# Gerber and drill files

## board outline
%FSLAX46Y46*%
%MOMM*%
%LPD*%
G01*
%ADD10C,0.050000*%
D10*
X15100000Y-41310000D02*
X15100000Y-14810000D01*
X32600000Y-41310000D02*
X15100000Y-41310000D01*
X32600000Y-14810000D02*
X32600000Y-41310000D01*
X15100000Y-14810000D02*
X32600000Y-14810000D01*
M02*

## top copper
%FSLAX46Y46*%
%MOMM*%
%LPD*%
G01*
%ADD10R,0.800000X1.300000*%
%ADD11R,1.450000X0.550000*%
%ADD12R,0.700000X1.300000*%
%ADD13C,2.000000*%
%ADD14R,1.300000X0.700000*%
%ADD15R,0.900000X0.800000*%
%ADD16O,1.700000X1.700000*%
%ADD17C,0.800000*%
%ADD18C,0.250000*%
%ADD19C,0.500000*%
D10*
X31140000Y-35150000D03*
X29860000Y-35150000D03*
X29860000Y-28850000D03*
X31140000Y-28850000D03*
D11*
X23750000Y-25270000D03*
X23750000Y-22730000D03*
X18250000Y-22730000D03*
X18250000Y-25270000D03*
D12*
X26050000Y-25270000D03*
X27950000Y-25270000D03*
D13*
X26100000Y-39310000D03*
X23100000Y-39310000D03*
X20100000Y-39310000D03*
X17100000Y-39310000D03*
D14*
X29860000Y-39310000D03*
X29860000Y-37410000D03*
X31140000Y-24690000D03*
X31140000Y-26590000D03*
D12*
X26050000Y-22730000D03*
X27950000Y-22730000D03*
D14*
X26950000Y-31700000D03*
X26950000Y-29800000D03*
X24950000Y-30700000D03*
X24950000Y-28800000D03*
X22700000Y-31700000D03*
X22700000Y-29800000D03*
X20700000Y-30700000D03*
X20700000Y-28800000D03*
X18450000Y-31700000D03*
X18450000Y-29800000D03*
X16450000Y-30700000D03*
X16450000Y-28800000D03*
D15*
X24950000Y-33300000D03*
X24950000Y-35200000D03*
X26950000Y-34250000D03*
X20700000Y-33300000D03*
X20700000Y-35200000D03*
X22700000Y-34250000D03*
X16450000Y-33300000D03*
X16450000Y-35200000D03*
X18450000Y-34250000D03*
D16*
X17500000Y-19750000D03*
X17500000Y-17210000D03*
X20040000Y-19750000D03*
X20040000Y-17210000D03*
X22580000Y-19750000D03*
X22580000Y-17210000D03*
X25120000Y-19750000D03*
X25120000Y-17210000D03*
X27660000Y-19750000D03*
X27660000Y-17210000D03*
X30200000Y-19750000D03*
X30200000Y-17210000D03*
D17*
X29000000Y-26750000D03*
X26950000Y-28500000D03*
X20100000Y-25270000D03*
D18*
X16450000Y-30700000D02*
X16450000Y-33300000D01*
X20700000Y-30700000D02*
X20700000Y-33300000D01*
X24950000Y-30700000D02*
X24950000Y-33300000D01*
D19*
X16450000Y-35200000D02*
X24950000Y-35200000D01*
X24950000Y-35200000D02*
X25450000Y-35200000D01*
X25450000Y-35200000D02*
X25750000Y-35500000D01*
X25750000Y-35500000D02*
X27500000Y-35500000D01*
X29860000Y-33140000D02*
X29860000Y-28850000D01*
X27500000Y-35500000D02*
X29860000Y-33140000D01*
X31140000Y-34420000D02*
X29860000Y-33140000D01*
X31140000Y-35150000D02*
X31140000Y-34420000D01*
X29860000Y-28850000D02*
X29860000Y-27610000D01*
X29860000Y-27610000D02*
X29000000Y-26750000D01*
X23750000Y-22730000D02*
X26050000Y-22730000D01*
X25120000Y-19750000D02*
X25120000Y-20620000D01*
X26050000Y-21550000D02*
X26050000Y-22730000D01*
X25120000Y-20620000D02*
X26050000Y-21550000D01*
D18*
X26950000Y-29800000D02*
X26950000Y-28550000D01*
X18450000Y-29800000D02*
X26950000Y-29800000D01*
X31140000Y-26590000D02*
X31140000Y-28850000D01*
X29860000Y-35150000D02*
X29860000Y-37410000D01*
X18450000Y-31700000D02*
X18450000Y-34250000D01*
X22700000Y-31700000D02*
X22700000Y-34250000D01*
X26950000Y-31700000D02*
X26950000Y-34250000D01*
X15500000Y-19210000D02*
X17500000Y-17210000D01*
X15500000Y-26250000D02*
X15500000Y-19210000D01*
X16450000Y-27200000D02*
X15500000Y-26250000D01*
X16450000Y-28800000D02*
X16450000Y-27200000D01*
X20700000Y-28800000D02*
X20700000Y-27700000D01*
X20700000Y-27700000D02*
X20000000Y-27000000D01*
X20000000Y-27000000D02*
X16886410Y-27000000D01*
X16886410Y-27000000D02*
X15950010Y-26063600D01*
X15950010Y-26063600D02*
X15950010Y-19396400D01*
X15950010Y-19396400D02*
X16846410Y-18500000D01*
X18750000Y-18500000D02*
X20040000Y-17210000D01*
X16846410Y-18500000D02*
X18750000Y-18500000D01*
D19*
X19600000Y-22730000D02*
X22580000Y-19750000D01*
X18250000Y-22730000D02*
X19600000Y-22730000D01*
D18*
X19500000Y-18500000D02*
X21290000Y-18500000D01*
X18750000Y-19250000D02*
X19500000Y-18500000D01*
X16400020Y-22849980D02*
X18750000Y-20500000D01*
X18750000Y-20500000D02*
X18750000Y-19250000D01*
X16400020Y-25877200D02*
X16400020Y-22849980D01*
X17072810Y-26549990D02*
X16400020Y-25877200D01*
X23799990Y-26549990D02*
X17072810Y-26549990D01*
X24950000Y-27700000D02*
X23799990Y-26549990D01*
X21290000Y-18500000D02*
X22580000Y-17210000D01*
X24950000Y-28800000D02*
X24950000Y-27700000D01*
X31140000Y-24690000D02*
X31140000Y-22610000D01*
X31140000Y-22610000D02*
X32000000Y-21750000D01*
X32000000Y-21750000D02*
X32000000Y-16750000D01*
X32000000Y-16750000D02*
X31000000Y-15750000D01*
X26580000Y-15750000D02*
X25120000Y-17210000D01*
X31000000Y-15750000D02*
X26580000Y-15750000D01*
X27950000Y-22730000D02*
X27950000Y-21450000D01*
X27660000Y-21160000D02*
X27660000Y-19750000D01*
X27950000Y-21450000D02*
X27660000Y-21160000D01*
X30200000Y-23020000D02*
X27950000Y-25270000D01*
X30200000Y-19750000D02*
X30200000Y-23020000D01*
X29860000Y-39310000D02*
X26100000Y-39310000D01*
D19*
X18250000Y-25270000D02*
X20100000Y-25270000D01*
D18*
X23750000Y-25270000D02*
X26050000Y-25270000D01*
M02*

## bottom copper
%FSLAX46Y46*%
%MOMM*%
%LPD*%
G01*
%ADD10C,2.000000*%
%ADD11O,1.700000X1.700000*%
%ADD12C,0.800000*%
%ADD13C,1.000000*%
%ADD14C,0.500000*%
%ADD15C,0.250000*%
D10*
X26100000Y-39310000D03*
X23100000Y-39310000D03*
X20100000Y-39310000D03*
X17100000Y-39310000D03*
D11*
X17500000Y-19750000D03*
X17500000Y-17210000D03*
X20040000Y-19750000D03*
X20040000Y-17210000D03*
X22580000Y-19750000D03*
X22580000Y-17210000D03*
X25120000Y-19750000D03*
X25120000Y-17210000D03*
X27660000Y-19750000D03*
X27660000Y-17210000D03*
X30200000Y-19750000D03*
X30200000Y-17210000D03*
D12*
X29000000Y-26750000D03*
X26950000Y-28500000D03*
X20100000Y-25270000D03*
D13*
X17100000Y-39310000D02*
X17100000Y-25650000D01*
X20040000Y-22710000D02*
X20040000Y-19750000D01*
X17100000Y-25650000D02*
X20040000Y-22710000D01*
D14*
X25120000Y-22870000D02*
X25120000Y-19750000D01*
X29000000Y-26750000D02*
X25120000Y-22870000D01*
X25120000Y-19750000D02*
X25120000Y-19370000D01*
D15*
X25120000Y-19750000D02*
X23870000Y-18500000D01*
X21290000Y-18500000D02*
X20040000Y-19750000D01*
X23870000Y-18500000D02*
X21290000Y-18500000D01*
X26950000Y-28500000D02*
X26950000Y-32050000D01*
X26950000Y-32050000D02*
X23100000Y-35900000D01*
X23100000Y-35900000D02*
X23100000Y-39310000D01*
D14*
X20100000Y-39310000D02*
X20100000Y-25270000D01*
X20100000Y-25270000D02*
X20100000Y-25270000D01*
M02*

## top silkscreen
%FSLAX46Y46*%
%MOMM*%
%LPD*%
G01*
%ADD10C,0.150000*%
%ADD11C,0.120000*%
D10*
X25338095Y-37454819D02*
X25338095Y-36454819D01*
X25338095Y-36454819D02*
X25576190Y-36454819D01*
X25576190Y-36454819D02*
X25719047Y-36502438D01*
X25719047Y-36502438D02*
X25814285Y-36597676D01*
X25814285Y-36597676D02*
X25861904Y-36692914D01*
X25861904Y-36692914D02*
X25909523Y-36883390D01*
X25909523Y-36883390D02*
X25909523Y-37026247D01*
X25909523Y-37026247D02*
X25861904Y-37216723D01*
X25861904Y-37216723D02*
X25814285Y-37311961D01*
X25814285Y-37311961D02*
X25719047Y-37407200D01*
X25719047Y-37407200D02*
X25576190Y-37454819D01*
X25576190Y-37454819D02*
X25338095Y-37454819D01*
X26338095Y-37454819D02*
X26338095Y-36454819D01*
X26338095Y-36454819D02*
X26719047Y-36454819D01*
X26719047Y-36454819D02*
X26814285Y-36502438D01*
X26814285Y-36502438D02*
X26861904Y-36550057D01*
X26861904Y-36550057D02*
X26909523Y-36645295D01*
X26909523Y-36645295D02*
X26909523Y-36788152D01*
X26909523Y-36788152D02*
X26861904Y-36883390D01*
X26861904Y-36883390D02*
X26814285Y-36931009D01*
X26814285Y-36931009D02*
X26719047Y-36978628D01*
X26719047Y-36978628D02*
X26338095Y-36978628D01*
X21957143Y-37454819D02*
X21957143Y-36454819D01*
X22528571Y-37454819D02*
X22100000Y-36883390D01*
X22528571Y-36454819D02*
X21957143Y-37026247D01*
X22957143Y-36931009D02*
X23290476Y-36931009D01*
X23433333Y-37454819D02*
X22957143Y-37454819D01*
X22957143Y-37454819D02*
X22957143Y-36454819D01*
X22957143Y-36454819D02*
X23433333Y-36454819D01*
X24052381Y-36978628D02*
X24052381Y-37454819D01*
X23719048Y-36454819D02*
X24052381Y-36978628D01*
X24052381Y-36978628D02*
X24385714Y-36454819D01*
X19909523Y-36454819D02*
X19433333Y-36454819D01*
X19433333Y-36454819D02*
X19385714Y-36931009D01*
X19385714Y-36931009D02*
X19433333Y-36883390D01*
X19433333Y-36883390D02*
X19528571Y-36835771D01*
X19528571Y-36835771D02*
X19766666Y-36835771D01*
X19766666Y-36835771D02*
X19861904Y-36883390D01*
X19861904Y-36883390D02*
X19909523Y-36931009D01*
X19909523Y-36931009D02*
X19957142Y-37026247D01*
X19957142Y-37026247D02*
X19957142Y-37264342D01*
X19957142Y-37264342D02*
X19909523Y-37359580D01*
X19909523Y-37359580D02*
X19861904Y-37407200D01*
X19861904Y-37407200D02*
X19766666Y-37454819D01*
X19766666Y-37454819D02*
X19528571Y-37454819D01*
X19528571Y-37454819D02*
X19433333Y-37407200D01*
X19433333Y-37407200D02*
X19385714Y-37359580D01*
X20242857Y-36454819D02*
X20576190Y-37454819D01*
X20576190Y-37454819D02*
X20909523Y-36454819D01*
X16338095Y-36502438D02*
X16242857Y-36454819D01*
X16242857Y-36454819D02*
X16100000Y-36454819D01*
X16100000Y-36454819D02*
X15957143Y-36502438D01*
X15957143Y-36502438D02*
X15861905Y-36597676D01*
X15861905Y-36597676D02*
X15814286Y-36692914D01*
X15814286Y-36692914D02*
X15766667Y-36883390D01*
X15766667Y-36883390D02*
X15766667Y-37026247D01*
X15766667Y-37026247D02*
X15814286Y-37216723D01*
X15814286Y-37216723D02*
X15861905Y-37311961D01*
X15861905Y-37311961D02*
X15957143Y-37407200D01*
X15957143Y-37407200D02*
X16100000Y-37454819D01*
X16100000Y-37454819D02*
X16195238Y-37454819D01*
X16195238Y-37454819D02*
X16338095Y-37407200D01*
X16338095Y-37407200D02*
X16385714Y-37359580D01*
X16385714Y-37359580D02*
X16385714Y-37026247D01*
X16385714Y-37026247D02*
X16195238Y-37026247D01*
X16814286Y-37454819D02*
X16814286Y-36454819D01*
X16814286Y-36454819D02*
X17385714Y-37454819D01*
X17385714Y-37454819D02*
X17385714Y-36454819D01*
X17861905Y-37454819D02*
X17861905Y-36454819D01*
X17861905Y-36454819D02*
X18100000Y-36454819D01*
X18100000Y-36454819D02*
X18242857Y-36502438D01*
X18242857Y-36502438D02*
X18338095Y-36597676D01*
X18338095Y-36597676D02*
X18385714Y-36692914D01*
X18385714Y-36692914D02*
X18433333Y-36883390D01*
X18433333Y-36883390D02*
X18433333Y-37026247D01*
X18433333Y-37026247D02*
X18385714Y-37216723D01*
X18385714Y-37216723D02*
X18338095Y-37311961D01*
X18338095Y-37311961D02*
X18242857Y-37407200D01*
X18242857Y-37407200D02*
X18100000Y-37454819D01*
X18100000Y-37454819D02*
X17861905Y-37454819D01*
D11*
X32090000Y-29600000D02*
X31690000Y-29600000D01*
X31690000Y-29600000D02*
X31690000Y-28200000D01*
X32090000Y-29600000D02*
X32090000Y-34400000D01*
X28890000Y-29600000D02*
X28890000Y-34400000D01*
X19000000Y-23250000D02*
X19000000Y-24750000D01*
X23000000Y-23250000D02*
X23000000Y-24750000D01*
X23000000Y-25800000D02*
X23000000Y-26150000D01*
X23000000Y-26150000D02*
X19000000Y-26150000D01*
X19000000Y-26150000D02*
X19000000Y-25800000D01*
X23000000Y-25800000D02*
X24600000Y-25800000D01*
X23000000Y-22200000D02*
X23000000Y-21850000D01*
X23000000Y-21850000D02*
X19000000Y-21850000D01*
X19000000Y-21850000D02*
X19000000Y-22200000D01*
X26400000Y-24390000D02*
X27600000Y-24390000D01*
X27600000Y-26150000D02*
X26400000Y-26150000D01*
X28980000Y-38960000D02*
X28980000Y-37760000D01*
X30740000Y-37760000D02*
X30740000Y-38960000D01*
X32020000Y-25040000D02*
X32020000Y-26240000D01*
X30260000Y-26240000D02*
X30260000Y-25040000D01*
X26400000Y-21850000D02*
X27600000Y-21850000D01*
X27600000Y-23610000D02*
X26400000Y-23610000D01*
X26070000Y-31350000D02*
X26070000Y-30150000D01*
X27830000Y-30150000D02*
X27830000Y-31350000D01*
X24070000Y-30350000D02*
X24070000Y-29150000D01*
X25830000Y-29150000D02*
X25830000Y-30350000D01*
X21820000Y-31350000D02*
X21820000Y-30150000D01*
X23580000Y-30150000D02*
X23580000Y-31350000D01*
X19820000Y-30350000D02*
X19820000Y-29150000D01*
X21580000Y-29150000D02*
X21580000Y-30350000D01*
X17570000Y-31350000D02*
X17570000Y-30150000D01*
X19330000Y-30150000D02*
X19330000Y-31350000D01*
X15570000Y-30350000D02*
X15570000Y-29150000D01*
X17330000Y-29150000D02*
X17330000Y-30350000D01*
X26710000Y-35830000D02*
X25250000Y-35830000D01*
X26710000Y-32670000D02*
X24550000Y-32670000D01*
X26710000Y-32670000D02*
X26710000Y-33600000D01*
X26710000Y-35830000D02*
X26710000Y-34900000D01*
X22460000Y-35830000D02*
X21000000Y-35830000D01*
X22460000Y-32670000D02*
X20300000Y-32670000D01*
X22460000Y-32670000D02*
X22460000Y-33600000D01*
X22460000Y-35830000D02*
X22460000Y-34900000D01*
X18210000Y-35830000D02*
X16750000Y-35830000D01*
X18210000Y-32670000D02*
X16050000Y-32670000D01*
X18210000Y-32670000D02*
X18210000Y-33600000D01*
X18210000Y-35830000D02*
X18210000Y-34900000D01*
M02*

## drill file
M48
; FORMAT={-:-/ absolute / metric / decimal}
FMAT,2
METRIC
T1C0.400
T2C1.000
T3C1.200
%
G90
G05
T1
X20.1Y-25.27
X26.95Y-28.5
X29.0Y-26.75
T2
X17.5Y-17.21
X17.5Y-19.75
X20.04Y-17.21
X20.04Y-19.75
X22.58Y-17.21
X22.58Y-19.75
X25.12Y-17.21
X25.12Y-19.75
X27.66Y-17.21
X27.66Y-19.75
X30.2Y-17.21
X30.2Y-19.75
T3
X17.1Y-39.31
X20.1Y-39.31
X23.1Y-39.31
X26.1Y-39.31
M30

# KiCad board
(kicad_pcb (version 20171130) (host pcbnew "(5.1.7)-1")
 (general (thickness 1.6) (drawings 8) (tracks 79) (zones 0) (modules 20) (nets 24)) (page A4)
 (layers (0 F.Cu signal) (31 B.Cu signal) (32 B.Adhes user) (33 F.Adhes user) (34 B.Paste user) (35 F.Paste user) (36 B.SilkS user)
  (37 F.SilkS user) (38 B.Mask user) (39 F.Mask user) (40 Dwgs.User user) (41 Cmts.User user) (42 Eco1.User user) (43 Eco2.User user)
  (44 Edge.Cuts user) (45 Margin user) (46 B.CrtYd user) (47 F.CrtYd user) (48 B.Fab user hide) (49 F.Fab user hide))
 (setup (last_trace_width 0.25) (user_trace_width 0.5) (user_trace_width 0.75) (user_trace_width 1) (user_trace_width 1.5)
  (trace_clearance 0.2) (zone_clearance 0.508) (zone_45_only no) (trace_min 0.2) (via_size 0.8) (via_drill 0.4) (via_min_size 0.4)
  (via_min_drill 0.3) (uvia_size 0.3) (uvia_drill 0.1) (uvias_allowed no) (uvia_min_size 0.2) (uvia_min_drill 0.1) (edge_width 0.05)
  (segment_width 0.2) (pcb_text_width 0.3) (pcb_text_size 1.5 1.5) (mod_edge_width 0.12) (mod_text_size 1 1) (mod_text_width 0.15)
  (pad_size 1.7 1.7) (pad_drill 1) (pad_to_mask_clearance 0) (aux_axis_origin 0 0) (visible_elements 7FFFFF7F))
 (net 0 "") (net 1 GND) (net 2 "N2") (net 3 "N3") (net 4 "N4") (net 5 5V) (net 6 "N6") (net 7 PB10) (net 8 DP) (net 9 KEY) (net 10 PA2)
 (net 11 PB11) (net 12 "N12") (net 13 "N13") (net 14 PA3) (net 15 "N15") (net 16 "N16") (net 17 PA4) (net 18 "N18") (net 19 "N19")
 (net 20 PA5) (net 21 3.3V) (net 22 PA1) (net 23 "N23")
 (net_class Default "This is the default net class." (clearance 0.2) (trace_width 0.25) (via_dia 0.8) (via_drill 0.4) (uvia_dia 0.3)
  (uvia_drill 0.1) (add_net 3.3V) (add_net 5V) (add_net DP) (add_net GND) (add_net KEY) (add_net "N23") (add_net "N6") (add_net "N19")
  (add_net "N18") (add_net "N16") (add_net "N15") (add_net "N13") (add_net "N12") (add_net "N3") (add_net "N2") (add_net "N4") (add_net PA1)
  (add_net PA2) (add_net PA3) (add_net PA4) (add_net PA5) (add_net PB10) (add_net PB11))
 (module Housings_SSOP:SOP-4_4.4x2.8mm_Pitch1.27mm (layer F.Cu) (at 30.5 32 270)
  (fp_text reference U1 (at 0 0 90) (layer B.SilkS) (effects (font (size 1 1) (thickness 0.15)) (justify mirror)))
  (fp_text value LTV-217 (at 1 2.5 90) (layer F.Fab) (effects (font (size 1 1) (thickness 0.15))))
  (fp_line (start -2.4 -1.59) (end -2.4 -1.19) (layer F.SilkS) (width 0.12))
  (fp_line (start -2.4 -1.19) (end -3.8 -1.19) (layer F.SilkS) (width 0.12))
  (fp_line (start -2.4 -1.59) (end 2.4 -1.59) (layer F.SilkS) (width 0.12))
  (fp_line (start -2.4 1.61) (end 2.4 1.61) (layer F.SilkS) (width 0.12))
  (pad 4 smd rect (at 3.15 -0.64 270) (size 1.3 0.8) (layers F.Cu F.Paste F.Mask) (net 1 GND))
  (pad 3 smd rect (at 3.15 0.64 270) (size 1.3 0.8) (layers F.Cu F.Paste F.Mask) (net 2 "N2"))
  (pad 2 smd rect (at -3.15 0.64 270) (size 1.3 0.8) (layers F.Cu F.Paste F.Mask) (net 1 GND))
  (pad 1 smd rect (at -3.15 -0.64 270) (size 1.3 0.8) (layers F.Cu F.Paste F.Mask) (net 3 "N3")))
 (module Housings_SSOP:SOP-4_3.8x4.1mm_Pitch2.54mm (layer F.Cu) (at 21 24 180)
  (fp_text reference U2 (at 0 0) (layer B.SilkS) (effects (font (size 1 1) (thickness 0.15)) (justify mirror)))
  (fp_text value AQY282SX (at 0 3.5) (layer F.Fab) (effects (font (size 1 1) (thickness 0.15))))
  (fp_line (start 2 0.75) (end 2 -0.75) (layer F.SilkS) (width 0.12))
  (fp_line (start -2 0.75) (end -2 -0.75) (layer F.SilkS) (width 0.12))
  (fp_line (start -2 -1.8) (end -2 -2.15) (layer F.SilkS) (width 0.12))
  (fp_line (start -2 -2.15) (end 2 -2.15) (layer F.SilkS) (width 0.12))
  (fp_line (start 2 -2.15) (end 2 -1.8) (layer F.SilkS) (width 0.12))
  (fp_line (start -2 -1.8) (end -3.6 -1.8) (layer F.SilkS) (width 0.12))
  (fp_line (start -2 1.8) (end -2 2.15) (layer F.SilkS) (width 0.12))
  (fp_line (start -2 2.15) (end 2 2.15) (layer F.SilkS) (width 0.12))
  (fp_line (start 2 2.15) (end 2 1.8) (layer F.SilkS) (width 0.12))
  (pad 1 smd rect (at -2.75 -1.27 180) (size 1.45 0.55) (layers F.Cu F.Paste F.Mask) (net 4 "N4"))
  (pad 2 smd rect (at -2.75 1.27 180) (size 1.45 0.55) (layers F.Cu F.Paste F.Mask) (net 1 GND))
  (pad 3 smd rect (at 2.75 1.27 180) (size 1.45 0.55) (layers F.Cu F.Paste F.Mask) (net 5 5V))
  (pad 4 smd rect (at 2.75 -1.27 180) (size 1.45 0.55) (layers F.Cu F.Paste F.Mask) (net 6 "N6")))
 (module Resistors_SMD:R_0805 (layer F.Cu) (at 27 25.27)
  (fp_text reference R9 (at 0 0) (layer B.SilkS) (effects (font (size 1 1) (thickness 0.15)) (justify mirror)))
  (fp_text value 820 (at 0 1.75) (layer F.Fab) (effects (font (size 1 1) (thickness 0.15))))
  (fp_line (start -0.6 -0.88) (end 0.6 -0.88) (layer F.SilkS) (width 0.12))
  (fp_line (start 0.6 0.88) (end -0.6 0.88) (layer F.SilkS) (width 0.12))
  (pad 1 smd rect (at -0.95 0) (size 0.7 1.3) (layers F.Cu F.Paste F.Mask) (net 4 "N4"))
  (pad 2 smd rect (at 0.95 0) (size 0.7 1.3) (layers F.Cu F.Paste F.Mask) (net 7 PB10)))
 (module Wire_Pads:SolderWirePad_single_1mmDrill (layer F.Cu) (at 26.1 39.31)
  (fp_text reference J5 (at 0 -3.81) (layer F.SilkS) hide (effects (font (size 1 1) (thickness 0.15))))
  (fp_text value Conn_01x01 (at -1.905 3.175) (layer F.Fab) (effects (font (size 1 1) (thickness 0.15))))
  (pad 1 thru_hole circle (at 0 0) (size 2 2) (drill 1.2) (layers *.Cu *.Mask) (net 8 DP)))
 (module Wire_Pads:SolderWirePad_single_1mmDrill (layer F.Cu) (at 23.1 39.31)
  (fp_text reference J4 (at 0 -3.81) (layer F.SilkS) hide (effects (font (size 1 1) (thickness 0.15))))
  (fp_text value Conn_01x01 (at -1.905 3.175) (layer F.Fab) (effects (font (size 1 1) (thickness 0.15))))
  (pad 1 thru_hole circle (at 0 0) (size 2 2) (drill 1.2) (layers *.Cu *.Mask) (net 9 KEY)))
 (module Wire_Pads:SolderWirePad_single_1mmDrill (layer F.Cu) (at 20.1 39.31)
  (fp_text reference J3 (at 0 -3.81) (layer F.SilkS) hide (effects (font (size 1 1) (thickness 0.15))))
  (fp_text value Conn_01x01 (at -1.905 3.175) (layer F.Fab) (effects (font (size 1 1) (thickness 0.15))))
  (pad 1 thru_hole circle (at 0 0) (size 2 2) (drill 1.2) (layers *.Cu *.Mask) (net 6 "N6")))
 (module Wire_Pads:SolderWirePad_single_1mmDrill (layer F.Cu) (at 17.1 39.31)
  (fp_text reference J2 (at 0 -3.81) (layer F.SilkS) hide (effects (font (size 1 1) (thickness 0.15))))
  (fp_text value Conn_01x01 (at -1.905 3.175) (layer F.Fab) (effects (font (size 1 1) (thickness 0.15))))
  (pad 1 thru_hole circle (at 0 0) (size 2 2) (drill 1.2) (layers *.Cu *.Mask) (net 1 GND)))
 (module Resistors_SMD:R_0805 (layer F.Cu) (at 29.86 38.36 90)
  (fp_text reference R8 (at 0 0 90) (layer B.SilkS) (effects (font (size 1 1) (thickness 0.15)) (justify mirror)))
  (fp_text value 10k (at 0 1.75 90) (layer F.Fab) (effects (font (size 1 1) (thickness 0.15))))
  (fp_line (start -0.6 -0.88) (end 0.6 -0.88) (layer F.SilkS) (width 0.12))
  (fp_line (start 0.6 0.88) (end -0.6 0.88) (layer F.SilkS) (width 0.12))
  (pad 1 smd rect (at -0.95 0 90) (size 0.7 1.3) (layers F.Cu F.Paste F.Mask) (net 8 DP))
  (pad 2 smd rect (at 0.95 0 90) (size 0.7 1.3) (layers F.Cu F.Paste F.Mask) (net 2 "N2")))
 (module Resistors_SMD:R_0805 (layer F.Cu) (at 31.14 25.64 90)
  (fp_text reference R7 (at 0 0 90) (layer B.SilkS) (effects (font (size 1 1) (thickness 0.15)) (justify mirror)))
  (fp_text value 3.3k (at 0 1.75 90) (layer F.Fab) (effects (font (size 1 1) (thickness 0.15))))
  (fp_line (start 0.6 0.88) (end -0.6 0.88) (layer F.SilkS) (width 0.12))
  (fp_line (start -0.6 -0.88) (end 0.6 -0.88) (layer F.SilkS) (width 0.12))
  (pad 2 smd rect (at 0.95 0 90) (size 0.7 1.3) (layers F.Cu F.Paste F.Mask) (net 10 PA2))
  (pad 1 smd rect (at -0.95 0 90) (size 0.7 1.3) (layers F.Cu F.Paste F.Mask) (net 3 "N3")))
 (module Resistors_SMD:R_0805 (layer F.Cu) (at 27 22.73)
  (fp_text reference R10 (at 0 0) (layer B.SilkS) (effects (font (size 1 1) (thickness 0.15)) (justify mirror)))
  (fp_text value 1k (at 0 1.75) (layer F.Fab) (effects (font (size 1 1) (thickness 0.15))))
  (fp_line (start -0.6 -0.88) (end 0.6 -0.88) (layer F.SilkS) (width 0.12))
  (fp_line (start 0.6 0.88) (end -0.6 0.88) (layer F.SilkS) (width 0.12))
  (pad 1 smd rect (at -0.95 0) (size 0.7 1.3) (layers F.Cu F.Paste F.Mask) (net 1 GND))
  (pad 2 smd rect (at 0.95 0) (size 0.7 1.3) (layers F.Cu F.Paste F.Mask) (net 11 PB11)))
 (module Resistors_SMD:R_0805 (layer F.Cu) (at 26.95 30.75 90)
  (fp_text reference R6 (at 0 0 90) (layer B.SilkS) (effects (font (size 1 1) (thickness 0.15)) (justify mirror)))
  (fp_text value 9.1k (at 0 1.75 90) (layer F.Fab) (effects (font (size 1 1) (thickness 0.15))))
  (fp_line (start -0.6 -0.88) (end 0.6 -0.88) (layer F.SilkS) (width 0.12))
  (fp_line (start 0.6 0.88) (end -0.6 0.88) (layer F.SilkS) (width 0.12))
  (pad 1 smd rect (at -0.95 0 90) (size 0.7 1.3) (layers F.Cu F.Paste F.Mask) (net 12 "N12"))
  (pad 2 smd rect (at 0.95 0 90) (size 0.7 1.3) (layers F.Cu F.Paste F.Mask) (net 9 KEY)))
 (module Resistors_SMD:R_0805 (layer F.Cu) (at 24.95 29.75 90)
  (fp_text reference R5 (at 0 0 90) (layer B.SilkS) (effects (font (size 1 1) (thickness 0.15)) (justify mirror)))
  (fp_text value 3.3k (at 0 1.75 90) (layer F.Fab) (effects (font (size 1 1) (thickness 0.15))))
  (fp_line (start -0.6 -0.88) (end 0.6 -0.88) (layer F.SilkS) (width 0.12))
  (fp_line (start 0.6 0.88) (end -0.6 0.88) (layer F.SilkS) (width 0.12))
  (pad 1 smd rect (at -0.95 0 90) (size 0.7 1.3) (layers F.Cu F.Paste F.Mask) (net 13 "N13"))
  (pad 2 smd rect (at 0.95 0 90) (size 0.7 1.3) (layers F.Cu F.Paste F.Mask) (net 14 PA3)))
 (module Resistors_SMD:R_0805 (layer F.Cu) (at 22.7 30.75 90)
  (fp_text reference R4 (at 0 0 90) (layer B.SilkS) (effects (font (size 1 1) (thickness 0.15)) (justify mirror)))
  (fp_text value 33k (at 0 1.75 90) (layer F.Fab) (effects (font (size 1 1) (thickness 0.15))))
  (fp_line (start -0.6 -0.88) (end 0.6 -0.88) (layer F.SilkS) (width 0.12))
  (fp_line (start 0.6 0.88) (end -0.6 0.88) (layer F.SilkS) (width 0.12))
  (pad 1 smd rect (at -0.95 0 90) (size 0.7 1.3) (layers F.Cu F.Paste F.Mask) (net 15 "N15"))
  (pad 2 smd rect (at 0.95 0 90) (size 0.7 1.3) (layers F.Cu F.Paste F.Mask) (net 9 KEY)))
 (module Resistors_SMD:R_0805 (layer F.Cu) (at 20.7 29.75 90)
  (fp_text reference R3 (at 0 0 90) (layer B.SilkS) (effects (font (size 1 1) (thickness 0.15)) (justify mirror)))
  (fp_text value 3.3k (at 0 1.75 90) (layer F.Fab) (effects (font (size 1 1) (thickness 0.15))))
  (fp_line (start -0.6 -0.88) (end 0.6 -0.88) (layer F.SilkS) (width 0.12))
  (fp_line (start 0.6 0.88) (end -0.6 0.88) (layer F.SilkS) (width 0.12))
  (pad 1 smd rect (at -0.95 0 90) (size 0.7 1.3) (layers F.Cu F.Paste F.Mask) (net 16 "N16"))
  (pad 2 smd rect (at 0.95 0 90) (size 0.7 1.3) (layers F.Cu F.Paste F.Mask) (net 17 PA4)))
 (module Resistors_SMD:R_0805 (layer F.Cu) (at 18.45 30.75 90)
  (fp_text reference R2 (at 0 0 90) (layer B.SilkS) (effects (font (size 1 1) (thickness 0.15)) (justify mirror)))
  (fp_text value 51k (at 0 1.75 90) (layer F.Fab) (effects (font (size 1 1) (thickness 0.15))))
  (fp_line (start -0.6 -0.88) (end 0.6 -0.88) (layer F.SilkS) (width 0.12))
  (fp_line (start 0.6 0.88) (end -0.6 0.88) (layer F.SilkS) (width 0.12))
  (pad 1 smd rect (at -0.95 0 90) (size 0.7 1.3) (layers F.Cu F.Paste F.Mask) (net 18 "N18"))
  (pad 2 smd rect (at 0.95 0 90) (size 0.7 1.3) (layers F.Cu F.Paste F.Mask) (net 9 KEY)))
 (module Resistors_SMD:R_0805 (layer F.Cu) (at 16.45 29.75 90)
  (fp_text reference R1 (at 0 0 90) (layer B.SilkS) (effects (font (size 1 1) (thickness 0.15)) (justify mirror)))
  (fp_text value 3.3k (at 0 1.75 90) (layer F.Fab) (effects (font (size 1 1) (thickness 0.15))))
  (fp_line (start -0.6 -0.88) (end 0.6 -0.88) (layer F.SilkS) (width 0.12))
  (fp_line (start 0.6 0.88) (end -0.6 0.88) (layer F.SilkS) (width 0.12))
  (pad 1 smd rect (at -0.95 0 90) (size 0.7 1.3) (layers F.Cu F.Paste F.Mask) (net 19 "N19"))
  (pad 2 smd rect (at 0.95 0 90) (size 0.7 1.3) (layers F.Cu F.Paste F.Mask) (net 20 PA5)))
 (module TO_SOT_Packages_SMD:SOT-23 (layer F.Cu) (at 25.95 34.25)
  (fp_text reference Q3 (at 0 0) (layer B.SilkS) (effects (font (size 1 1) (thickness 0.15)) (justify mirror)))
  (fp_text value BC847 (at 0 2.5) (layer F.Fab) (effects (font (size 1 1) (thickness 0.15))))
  (fp_line (start 0.76 1.58) (end -0.7 1.58) (layer F.SilkS) (width 0.12))
  (fp_line (start 0.76 -1.58) (end -1.4 -1.58) (layer F.SilkS) (width 0.12))
  (fp_line (start 0.76 -1.58) (end 0.76 -0.65) (layer F.SilkS) (width 0.12))
  (fp_line (start 0.76 1.58) (end 0.76 0.65) (layer F.SilkS) (width 0.12))
  (pad 1 smd rect (at -1 -0.95) (size 0.9 0.8) (layers F.Cu F.Paste F.Mask) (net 13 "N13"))
  (pad 2 smd rect (at -1 0.95) (size 0.9 0.8) (layers F.Cu F.Paste F.Mask) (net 1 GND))
  (pad 3 smd rect (at 1 0) (size 0.9 0.8) (layers F.Cu F.Paste F.Mask) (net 12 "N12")))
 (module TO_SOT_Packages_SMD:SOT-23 (layer F.Cu) (at 21.7 34.25)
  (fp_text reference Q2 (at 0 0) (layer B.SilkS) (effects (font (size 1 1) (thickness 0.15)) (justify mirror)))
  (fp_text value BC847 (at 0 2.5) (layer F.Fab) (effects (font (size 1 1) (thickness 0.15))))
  (fp_line (start 0.76 1.58) (end -0.7 1.58) (layer F.SilkS) (width 0.12))
  (fp_line (start 0.76 -1.58) (end -1.4 -1.58) (layer F.SilkS) (width 0.12))
  (fp_line (start 0.76 -1.58) (end 0.76 -0.65) (layer F.SilkS) (width 0.12))
  (fp_line (start 0.76 1.58) (end 0.76 0.65) (layer F.SilkS) (width 0.12))
  (pad 1 smd rect (at -1 -0.95) (size 0.9 0.8) (layers F.Cu F.Paste F.Mask) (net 16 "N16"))
  (pad 2 smd rect (at -1 0.95) (size 0.9 0.8) (layers F.Cu F.Paste F.Mask) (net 1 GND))
  (pad 3 smd rect (at 1 0) (size 0.9 0.8) (layers F.Cu F.Paste F.Mask) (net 15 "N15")))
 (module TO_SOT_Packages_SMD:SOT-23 (layer F.Cu) (at 17.45 34.25)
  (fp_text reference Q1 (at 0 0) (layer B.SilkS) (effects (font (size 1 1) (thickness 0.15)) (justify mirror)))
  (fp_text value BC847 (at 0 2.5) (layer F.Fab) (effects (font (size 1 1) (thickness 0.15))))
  (fp_line (start 0.76 1.58) (end -0.7 1.58) (layer F.SilkS) (width 0.12))
  (fp_line (start 0.76 -1.58) (end -1.4 -1.58) (layer F.SilkS) (width 0.12))
  (fp_line (start 0.76 -1.58) (end 0.76 -0.65) (layer F.SilkS) (width 0.12))
  (fp_line (start 0.76 1.58) (end 0.76 0.65) (layer F.SilkS) (width 0.12))
  (pad 1 smd rect (at -1 -0.95) (size 0.9 0.8) (layers F.Cu F.Paste F.Mask) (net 19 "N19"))
  (pad 2 smd rect (at -1 0.95) (size 0.9 0.8) (layers F.Cu F.Paste F.Mask) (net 1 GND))
  (pad 3 smd rect (at 1 0) (size 0.9 0.8) (layers F.Cu F.Paste F.Mask) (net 18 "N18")))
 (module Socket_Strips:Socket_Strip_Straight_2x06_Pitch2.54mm (layer B.Cu) (at 17.5 19.75 270)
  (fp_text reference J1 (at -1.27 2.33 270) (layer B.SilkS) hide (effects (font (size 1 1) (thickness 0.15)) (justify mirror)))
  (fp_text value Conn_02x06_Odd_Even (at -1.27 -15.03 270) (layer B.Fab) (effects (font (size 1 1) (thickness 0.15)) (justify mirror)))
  (pad 1 thru_hole oval (at 0 0 270) (size 1.7 1.7) (drill 1) (layers *.Cu *.Mask) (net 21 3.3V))
  (pad 2 thru_hole oval (at -2.54 0 270) (size 1.7 1.7) (drill 1) (layers *.Cu *.Mask) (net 20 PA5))
  (pad 3 thru_hole oval (at 0 -2.54 270) (size 1.7 1.7) (drill 1) (layers *.Cu *.Mask) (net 1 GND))
  (pad 4 thru_hole oval (at -2.54 -2.54 270) (size 1.7 1.7) (drill 1) (layers *.Cu *.Mask) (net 17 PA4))
  (pad 5 thru_hole oval (at 0 -5.08 270) (size 1.7 1.7) (drill 1) (layers *.Cu *.Mask) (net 5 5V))
  (pad 6 thru_hole oval (at -2.54 -5.08 270) (size 1.7 1.7) (drill 1) (layers *.Cu *.Mask) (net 14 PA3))
  (pad 7 thru_hole oval (at 0 -7.62 270) (size 1.7 1.7) (drill 1) (layers *.Cu *.Mask) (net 1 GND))
  (pad 8 thru_hole oval (at -2.54 -7.62 270) (size 1.7 1.7) (drill 1) (layers *.Cu *.Mask) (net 10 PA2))
  (pad 9 thru_hole oval (at 0 -10.16 270) (size 1.7 1.7) (drill 1) (layers *.Cu *.Mask) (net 11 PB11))
  (pad 10 thru_hole oval (at -2.54 -10.16 270) (size 1.7 1.7) (drill 1) (layers *.Cu *.Mask) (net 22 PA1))
  (pad 11 thru_hole oval (at 0 -12.7 270) (size 1.7 1.7) (drill 1) (layers *.Cu *.Mask) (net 7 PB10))
  (pad 12 thru_hole oval (at -2.54 -12.7 270) (size 1.7 1.7) (drill 1) (layers *.Cu *.Mask) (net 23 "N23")))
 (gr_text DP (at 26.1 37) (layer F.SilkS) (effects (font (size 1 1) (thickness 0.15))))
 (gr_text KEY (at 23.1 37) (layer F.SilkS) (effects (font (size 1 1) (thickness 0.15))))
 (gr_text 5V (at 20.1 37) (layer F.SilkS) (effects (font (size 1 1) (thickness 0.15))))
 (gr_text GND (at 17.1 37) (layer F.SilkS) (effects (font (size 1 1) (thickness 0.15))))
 (gr_line (start 15.1 41.31) (end 15.1 14.81) (layer Edge.Cuts) (width 0.05))
 (gr_line (start 32.6 41.31) (end 15.1 41.31) (layer Edge.Cuts) (width 0.05))
 (gr_line (start 32.6 14.81) (end 32.6 41.31) (layer Edge.Cuts) (width 0.05))
 (gr_line (start 15.1 14.81) (end 32.6 14.81) (layer Edge.Cuts) (width 0.05))
 (segment (start 16.45 30.7) (end 16.45 33.3) (width 0.25) (layer F.Cu) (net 19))
 (segment (start 20.7 30.7) (end 20.7 33.3) (width 0.25) (layer F.Cu) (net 16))
 (segment (start 24.95 30.7) (end 24.95 33.3) (width 0.25) (layer F.Cu) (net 13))
 (segment (start 16.45 35.2) (end 24.95 35.2) (width 0.5) (layer F.Cu) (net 1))
 (segment (start 17.1 39.31) (end 17.1 25.65) (width 1) (layer B.Cu) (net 1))
 (segment (start 20.04 22.71) (end 20.04 19.75) (width 1) (layer B.Cu) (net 1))
 (segment (start 17.1 25.65) (end 20.04 22.71) (width 1) (layer B.Cu) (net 1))
 (segment (start 24.95 35.2) (end 25.45 35.2) (width 0.5) (layer F.Cu) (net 1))
 (segment (start 25.45 35.2) (end 25.75 35.5) (width 0.5) (layer F.Cu) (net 1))
 (segment (start 25.75 35.5) (end 27.5 35.5) (width 0.5) (layer F.Cu) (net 1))
 (segment (start 29.86 33.14) (end 29.86 28.85) (width 0.5) (layer F.Cu) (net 1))
 (segment (start 27.5 35.5) (end 29.86 33.14) (width 0.5) (layer F.Cu) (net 1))
 (segment (start 31.14 34.42) (end 29.86 33.14) (width 0.5) (layer F.Cu) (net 1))
 (segment (start 31.14 35.15) (end 31.14 34.42) (width 0.5) (layer F.Cu) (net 1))
 (segment (start 29.86 28.85) (end 29.86 27.61) (width 0.5) (layer F.Cu) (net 1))
 (segment (start 29.86 27.61) (end 29 26.75) (width 0.5) (layer F.Cu) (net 1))
 (via (at 29 26.75) (size 0.8) (drill 0.4) (layers F.Cu B.Cu) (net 1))
 (segment (start 25.12 22.87) (end 25.12 19.75) (width 0.5) (layer B.Cu) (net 1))
 (segment (start 29 26.75) (end 25.12 22.87) (width 0.5) (layer B.Cu) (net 1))
 (segment (start 25.12 19.75) (end 25.12 19.37) (width 0.5) (layer B.Cu) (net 1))
 (segment (start 25.12 19.75) (end 23.87 18.5) (width 0.25) (layer B.Cu) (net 1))
 (segment (start 21.29 18.5) (end 20.04 19.75) (width 0.25) (layer B.Cu) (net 1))
 (segment (start 23.87 18.5) (end 21.29 18.5) (width 0.25) (layer B.Cu) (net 1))
 (segment (start 23.75 22.73) (end 26.05 22.73) (width 0.5) (layer F.Cu) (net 1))
 (segment (start 25.12 19.75) (end 25.12 20.62) (width 0.5) (layer F.Cu) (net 1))
 (segment (start 26.05 21.55) (end 26.05 22.73) (width 0.5) (layer F.Cu) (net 1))
 (segment (start 25.12 20.62) (end 26.05 21.55) (width 0.5) (layer F.Cu) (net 1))
 (via (at 26.95 28.5) (size 0.8) (drill 0.4) (layers F.Cu B.Cu) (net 9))
 (segment (start 26.95 29.8) (end 26.95 28.55) (width 0.25) (layer F.Cu) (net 9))
 (segment (start 18.45 29.8) (end 26.95 29.8) (width 0.25) (layer F.Cu) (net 9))
 (segment (start 26.95 28.5) (end 26.95 32.05) (width 0.25) (layer B.Cu) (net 9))
 (segment (start 26.95 32.05) (end 23.1 35.9) (width 0.25) (layer B.Cu) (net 9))
 (segment (start 23.1 35.9) (end 23.1 39.31) (width 0.25) (layer B.Cu) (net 9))
 (segment (start 31.14 26.59) (end 31.14 28.85) (width 0.25) (layer F.Cu) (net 3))
 (segment (start 29.86 35.15) (end 29.86 37.41) (width 0.25) (layer F.Cu) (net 2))
 (segment (start 18.45 31.7) (end 18.45 34.25) (width 0.25) (layer F.Cu) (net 18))
 (segment (start 22.7 31.7) (end 22.7 34.25) (width 0.25) (layer F.Cu) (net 15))
 (segment (start 26.95 31.7) (end 26.95 34.25) (width 0.25) (layer F.Cu) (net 12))
 (segment (start 15.5 19.21) (end 17.5 17.21) (width 0.25) (layer F.Cu) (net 20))
 (segment (start 15.5 26.25) (end 15.5 19.21) (width 0.25) (layer F.Cu) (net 20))
 (segment (start 16.45 27.2) (end 15.5 26.25) (width 0.25) (layer F.Cu) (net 20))
 (segment (start 16.45 28.8) (end 16.45 27.2) (width 0.25) (layer F.Cu) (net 20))
 (segment (start 20.7 28.8) (end 20.7 27.7) (width 0.25) (layer F.Cu) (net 17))
 (segment (start 20.7 27.7) (end 20 27) (width 0.25) (layer F.Cu) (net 17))
 (segment (start 20 27) (end 16.88641 27) (width 0.25) (layer F.Cu) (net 17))
 (segment (start 16.88641 27) (end 15.95001 26.0636) (width 0.25) (layer F.Cu) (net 17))
 (segment (start 15.95001 26.0636) (end 15.95001 19.3964) (width 0.25) (layer F.Cu) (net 17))
 (segment (start 15.95001 19.3964) (end 16.84641 18.5) (width 0.25) (layer F.Cu) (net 17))
 (segment (start 18.75 18.5) (end 20.04 17.21) (width 0.25) (layer F.Cu) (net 17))
 (segment (start 16.84641 18.5) (end 18.75 18.5) (width 0.25) (layer F.Cu) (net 17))
 (segment (start 19.6 22.73) (end 22.58 19.75) (width 0.5) (layer F.Cu) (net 5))
 (segment (start 18.25 22.73) (end 19.6 22.73) (width 0.5) (layer F.Cu) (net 5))
 (segment (start 19.5 18.5) (end 21.29 18.5) (width 0.25) (layer F.Cu) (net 14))
 (segment (start 18.75 19.25) (end 19.5 18.5) (width 0.25) (layer F.Cu) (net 14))
 (segment (start 16.40002 22.84998) (end 18.75 20.5) (width 0.25) (layer F.Cu) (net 14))
 (segment (start 18.75 20.5) (end 18.75 19.25) (width 0.25) (layer F.Cu) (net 14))
 (segment (start 16.40002 25.8772) (end 16.40002 22.84998) (width 0.25) (layer F.Cu) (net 14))
 (segment (start 17.07281 26.54999) (end 16.40002 25.8772) (width 0.25) (layer F.Cu) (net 14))
 (segment (start 23.79999 26.54999) (end 17.07281 26.54999) (width 0.25) (layer F.Cu) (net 14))
 (segment (start 24.95 27.7) (end 23.79999 26.54999) (width 0.25) (layer F.Cu) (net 14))
 (segment (start 21.29 18.5) (end 22.58 17.21) (width 0.25) (layer F.Cu) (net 14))
 (segment (start 24.95 28.8) (end 24.95 27.7) (width 0.25) (layer F.Cu) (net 14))
 (segment (start 31.14 24.69) (end 31.14 22.61) (width 0.25) (layer F.Cu) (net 10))
 (segment (start 31.14 22.61) (end 32 21.75) (width 0.25) (layer F.Cu) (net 10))
 (segment (start 32 21.75) (end 32 16.75) (width 0.25) (layer F.Cu) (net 10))
 (segment (start 32 16.75) (end 31 15.75) (width 0.25) (layer F.Cu) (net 10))
 (segment (start 26.58 15.75) (end 25.12 17.21) (width 0.25) (layer F.Cu) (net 10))
 (segment (start 31 15.75) (end 26.58 15.75) (width 0.25) (layer F.Cu) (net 10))
 (segment (start 27.95 22.73) (end 27.95 21.45) (width 0.25) (layer F.Cu) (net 11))
 (segment (start 27.66 21.16) (end 27.66 19.75) (width 0.25) (layer F.Cu) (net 11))
 (segment (start 27.95 21.45) (end 27.66 21.16) (width 0.25) (layer F.Cu) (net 11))
 (segment (start 30.2 23.02) (end 27.95 25.27) (width 0.25) (layer F.Cu) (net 7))
 (segment (start 30.2 19.75) (end 30.2 23.02) (width 0.25) (layer F.Cu) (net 7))
 (segment (start 29.86 39.31) (end 26.1 39.31) (width 0.25) (layer F.Cu) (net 8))
 (segment (start 20.1 39.31) (end 20.1 25.27) (width 0.5) (layer B.Cu) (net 6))
 (segment (start 20.1 25.27) (end 20.1 25.27) (width 0.5) (layer B.Cu) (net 6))
 (via (at 20.1 25.27) (size 0.8) (drill 0.4) (layers F.Cu B.Cu) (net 6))
 (segment (start 18.25 25.27) (end 20.1 25.27) (width 0.5) (layer F.Cu) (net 6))
 (segment (start 23.75 25.27) (end 26.05 25.27) (width 0.25) (layer F.Cu) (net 4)))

